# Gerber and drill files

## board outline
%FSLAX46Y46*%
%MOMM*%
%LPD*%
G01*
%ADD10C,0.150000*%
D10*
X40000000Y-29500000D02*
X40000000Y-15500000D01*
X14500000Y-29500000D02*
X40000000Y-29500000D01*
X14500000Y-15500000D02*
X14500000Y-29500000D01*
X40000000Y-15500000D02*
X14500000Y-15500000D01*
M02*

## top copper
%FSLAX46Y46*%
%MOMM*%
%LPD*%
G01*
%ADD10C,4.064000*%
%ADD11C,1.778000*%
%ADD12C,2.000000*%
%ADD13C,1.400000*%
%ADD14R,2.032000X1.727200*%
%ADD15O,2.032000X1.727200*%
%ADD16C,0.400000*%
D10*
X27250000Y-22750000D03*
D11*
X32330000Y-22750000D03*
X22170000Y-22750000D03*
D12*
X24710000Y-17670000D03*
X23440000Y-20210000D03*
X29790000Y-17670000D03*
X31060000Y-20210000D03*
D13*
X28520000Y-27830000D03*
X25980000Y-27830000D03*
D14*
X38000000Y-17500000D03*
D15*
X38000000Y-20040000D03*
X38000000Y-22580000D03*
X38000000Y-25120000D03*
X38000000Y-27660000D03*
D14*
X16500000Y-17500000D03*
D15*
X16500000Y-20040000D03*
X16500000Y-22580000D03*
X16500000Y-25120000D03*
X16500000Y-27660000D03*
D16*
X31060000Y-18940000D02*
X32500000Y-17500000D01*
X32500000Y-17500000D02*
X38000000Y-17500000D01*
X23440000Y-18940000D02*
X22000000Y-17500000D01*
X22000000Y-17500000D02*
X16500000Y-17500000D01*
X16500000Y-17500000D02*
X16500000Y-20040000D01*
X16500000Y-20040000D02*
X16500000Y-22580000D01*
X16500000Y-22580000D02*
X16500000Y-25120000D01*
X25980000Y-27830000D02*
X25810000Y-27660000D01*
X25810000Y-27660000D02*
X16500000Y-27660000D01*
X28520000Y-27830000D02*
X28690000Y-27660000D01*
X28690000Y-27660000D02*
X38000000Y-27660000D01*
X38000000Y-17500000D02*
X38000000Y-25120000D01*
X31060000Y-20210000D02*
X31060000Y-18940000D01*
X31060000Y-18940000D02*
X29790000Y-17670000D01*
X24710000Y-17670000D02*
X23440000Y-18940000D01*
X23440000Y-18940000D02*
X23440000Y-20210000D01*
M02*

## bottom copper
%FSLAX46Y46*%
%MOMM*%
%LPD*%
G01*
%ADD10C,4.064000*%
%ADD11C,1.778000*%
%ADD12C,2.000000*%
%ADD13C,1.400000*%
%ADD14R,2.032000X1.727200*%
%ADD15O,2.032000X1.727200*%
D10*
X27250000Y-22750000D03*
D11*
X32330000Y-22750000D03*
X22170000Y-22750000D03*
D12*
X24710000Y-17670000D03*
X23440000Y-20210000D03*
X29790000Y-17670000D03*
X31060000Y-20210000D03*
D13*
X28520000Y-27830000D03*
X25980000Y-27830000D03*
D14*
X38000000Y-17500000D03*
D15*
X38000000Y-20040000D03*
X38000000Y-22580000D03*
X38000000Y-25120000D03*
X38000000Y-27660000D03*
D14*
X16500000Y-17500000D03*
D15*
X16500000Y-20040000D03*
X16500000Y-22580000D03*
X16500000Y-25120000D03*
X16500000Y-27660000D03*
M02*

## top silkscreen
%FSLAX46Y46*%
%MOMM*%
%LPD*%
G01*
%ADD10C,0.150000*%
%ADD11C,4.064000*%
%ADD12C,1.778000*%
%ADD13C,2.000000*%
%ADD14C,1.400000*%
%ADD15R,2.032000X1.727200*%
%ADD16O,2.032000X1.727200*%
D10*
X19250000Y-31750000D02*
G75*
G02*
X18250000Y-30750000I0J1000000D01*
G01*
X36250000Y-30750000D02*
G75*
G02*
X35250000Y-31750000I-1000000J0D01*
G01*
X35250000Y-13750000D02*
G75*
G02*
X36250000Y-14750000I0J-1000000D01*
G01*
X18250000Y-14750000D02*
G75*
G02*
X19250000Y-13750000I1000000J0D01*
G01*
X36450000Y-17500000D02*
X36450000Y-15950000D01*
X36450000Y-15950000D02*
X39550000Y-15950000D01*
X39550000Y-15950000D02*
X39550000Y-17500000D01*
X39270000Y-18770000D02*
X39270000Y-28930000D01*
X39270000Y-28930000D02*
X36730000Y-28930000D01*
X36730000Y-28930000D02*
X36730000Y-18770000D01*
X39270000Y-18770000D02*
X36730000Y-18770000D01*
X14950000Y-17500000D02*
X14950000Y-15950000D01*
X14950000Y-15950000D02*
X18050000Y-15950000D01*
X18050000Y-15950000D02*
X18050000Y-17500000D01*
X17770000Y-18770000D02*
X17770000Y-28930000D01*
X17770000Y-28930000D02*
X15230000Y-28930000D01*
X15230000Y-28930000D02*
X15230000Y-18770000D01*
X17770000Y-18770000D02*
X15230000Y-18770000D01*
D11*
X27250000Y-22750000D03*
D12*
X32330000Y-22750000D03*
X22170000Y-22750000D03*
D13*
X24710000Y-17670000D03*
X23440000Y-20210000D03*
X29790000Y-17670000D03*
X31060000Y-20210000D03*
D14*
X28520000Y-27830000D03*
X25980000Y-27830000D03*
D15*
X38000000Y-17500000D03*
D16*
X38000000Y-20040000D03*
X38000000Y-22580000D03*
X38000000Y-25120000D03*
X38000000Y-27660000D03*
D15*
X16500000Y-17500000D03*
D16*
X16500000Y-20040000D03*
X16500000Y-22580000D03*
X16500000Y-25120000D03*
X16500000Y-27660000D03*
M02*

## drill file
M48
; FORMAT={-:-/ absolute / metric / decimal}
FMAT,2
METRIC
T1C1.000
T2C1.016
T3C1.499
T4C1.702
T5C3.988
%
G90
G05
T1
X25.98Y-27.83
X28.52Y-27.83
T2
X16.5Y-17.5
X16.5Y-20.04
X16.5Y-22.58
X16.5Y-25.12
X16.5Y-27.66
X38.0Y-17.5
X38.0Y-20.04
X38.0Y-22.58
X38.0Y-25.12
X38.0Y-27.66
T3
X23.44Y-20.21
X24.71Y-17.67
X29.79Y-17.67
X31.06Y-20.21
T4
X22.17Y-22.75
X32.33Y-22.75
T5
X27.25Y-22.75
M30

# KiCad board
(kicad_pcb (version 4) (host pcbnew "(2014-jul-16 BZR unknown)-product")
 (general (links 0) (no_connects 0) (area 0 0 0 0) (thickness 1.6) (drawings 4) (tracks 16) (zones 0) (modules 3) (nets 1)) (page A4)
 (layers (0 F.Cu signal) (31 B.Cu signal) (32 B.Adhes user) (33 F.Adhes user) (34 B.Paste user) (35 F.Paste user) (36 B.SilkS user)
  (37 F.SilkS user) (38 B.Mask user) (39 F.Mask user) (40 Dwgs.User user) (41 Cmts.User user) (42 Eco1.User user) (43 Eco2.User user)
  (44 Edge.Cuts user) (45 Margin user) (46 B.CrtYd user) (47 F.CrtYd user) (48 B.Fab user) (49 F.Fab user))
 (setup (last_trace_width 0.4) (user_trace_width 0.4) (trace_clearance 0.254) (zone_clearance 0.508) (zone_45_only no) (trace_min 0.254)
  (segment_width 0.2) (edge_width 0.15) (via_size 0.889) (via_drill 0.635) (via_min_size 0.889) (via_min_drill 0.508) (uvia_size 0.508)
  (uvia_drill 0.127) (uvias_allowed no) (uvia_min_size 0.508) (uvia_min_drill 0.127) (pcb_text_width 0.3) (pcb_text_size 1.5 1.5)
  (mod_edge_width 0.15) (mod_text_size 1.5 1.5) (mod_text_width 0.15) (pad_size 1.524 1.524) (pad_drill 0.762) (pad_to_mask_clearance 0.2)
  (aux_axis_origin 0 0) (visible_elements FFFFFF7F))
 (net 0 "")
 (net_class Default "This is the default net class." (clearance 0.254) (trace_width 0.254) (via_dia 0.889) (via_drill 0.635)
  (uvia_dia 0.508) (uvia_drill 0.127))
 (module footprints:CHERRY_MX (layer F.Cu) (at 27.25 22.75)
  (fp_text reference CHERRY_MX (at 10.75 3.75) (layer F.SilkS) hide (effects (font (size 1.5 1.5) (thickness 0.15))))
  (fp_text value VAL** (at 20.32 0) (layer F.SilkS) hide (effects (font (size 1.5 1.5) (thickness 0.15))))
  (fp_arc (start -8 8) (end -8 9) (angle 90) (layer F.SilkS) (width 0.15))
  (fp_arc (start 8 8) (end 9 8) (angle 90) (layer F.SilkS) (width 0.15))
  (fp_arc (start 8 -8) (end 8 -9) (angle 90) (layer F.SilkS) (width 0.15))
  (fp_arc (start -8 -8) (end -9 -8) (angle 90) (layer F.SilkS) (width 0.15))
  (pad "" thru_hole circle (at 0 0) (size 4.064 4.064) (drill 3.9878) (layers *.Cu *.Mask F.SilkS))
  (pad "" thru_hole circle (at 5.08 0) (size 1.778 1.778) (drill 1.7018) (layers *.Cu *.Mask F.SilkS))
  (pad "" thru_hole circle (at -5.08 0) (size 1.778 1.778) (drill 1.7018) (layers *.Cu *.Mask F.SilkS))
  (pad 1 thru_hole circle (at -2.54 -5.08) (size 2 2) (drill 1.4986) (layers *.Cu *.Mask F.SilkS))
  (pad 1 thru_hole circle (at -3.81 -2.54) (size 2 2) (drill 1.4986) (layers *.Cu *.Mask F.SilkS))
  (pad 2 thru_hole circle (at 2.54 -5.08) (size 2 2) (drill 1.4986) (layers *.Cu *.Mask F.SilkS))
  (pad 2 thru_hole circle (at 3.81 -2.54) (size 2 2) (drill 1.4986) (layers *.Cu *.Mask F.SilkS))
  (pad 4 thru_hole circle (at 1.27 5.08) (size 1.4 1.4) (drill 1) (layers *.Cu *.Mask F.SilkS))
  (pad 3 thru_hole circle (at -1.27 5.08) (size 1.4 1.4) (drill 1) (layers *.Cu *.Mask F.SilkS)))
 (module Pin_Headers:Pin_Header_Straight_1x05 (layer F.Cu) (at 38 17.5)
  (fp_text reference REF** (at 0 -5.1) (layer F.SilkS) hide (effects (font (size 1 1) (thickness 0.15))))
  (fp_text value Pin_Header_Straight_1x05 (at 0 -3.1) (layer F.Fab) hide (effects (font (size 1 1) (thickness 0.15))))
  (fp_line (start -1.55 0) (end -1.55 -1.55) (layer F.SilkS) (width 0.15))
  (fp_line (start -1.55 -1.55) (end 1.55 -1.55) (layer F.SilkS) (width 0.15))
  (fp_line (start 1.55 -1.55) (end 1.55 0) (layer F.SilkS) (width 0.15))
  (fp_line (start 1.27 1.27) (end 1.27 11.43) (layer F.SilkS) (width 0.15))
  (fp_line (start 1.27 11.43) (end -1.27 11.43) (layer F.SilkS) (width 0.15))
  (fp_line (start -1.27 11.43) (end -1.27 1.27) (layer F.SilkS) (width 0.15))
  (fp_line (start 1.27 1.27) (end -1.27 1.27) (layer F.SilkS) (width 0.15))
  (pad 1 thru_hole rect (at 0 0) (size 2.032 1.7272) (drill 1.016) (layers *.Cu *.Mask F.SilkS))
  (pad 2 thru_hole oval (at 0 2.54) (size 2.032 1.7272) (drill 1.016) (layers *.Cu *.Mask F.SilkS))
  (pad 3 thru_hole oval (at 0 5.08) (size 2.032 1.7272) (drill 1.016) (layers *.Cu *.Mask F.SilkS))
  (pad 4 thru_hole oval (at 0 7.62) (size 2.032 1.7272) (drill 1.016) (layers *.Cu *.Mask F.SilkS))
  (pad 5 thru_hole oval (at 0 10.16) (size 2.032 1.7272) (drill 1.016) (layers *.Cu *.Mask F.SilkS)))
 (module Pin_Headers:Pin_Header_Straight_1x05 (layer F.Cu) (at 16.5 17.5)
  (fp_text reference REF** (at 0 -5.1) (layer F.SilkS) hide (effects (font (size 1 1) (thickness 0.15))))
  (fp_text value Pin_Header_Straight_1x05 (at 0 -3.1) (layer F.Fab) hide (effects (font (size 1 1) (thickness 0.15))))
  (fp_line (start -1.55 0) (end -1.55 -1.55) (layer F.SilkS) (width 0.15))
  (fp_line (start -1.55 -1.55) (end 1.55 -1.55) (layer F.SilkS) (width 0.15))
  (fp_line (start 1.55 -1.55) (end 1.55 0) (layer F.SilkS) (width 0.15))
  (fp_line (start 1.27 1.27) (end 1.27 11.43) (layer F.SilkS) (width 0.15))
  (fp_line (start 1.27 11.43) (end -1.27 11.43) (layer F.SilkS) (width 0.15))
  (fp_line (start -1.27 11.43) (end -1.27 1.27) (layer F.SilkS) (width 0.15))
  (fp_line (start 1.27 1.27) (end -1.27 1.27) (layer F.SilkS) (width 0.15))
  (pad 1 thru_hole rect (at 0 0) (size 2.032 1.7272) (drill 1.016) (layers *.Cu *.Mask F.SilkS))
  (pad 2 thru_hole oval (at 0 2.54) (size 2.032 1.7272) (drill 1.016) (layers *.Cu *.Mask F.SilkS))
  (pad 3 thru_hole oval (at 0 5.08) (size 2.032 1.7272) (drill 1.016) (layers *.Cu *.Mask F.SilkS))
  (pad 4 thru_hole oval (at 0 7.62) (size 2.032 1.7272) (drill 1.016) (layers *.Cu *.Mask F.SilkS))
  (pad 5 thru_hole oval (at 0 10.16) (size 2.032 1.7272) (drill 1.016) (layers *.Cu *.Mask F.SilkS)))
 (gr_line (start 40 29.5) (end 40 15.5) (angle 90) (layer Edge.Cuts) (width 0.15))
 (gr_line (start 14.5 29.5) (end 40 29.5) (angle 90) (layer Edge.Cuts) (width 0.15))
 (gr_line (start 14.5 15.5) (end 14.5 29.5) (angle 90) (layer Edge.Cuts) (width 0.15))
 (gr_line (start 40 15.5) (end 14.5 15.5) (angle 90) (layer Edge.Cuts) (width 0.15))
 (segment (start 31.06 18.94) (end 32.5 17.5) (width 0.4) (layer F.Cu) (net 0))
 (segment (start 32.5 17.5) (end 38 17.5) (width 0.4) (layer F.Cu) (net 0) (status 800000))
 (segment (start 23.44 18.94) (end 22 17.5) (width 0.4) (layer F.Cu) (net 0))
 (segment (start 22 17.5) (end 16.5 17.5) (width 0.4) (layer F.Cu) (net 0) (status 800000))
 (segment (start 16.5 17.5) (end 16.5 20.04) (width 0.4) (layer F.Cu) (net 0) (status C00000))
 (segment (start 16.5 20.04) (end 16.5 22.58) (width 0.4) (layer F.Cu) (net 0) (status C00000))
 (segment (start 16.5 22.58) (end 16.5 25.12) (width 0.4) (layer F.Cu) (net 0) (status C00000))
 (segment (start 25.98 27.83) (end 25.81 27.66) (width 0.4) (layer F.Cu) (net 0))
 (segment (start 25.81 27.66) (end 16.5 27.66) (width 0.4) (layer F.Cu) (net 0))
 (segment (start 28.52 27.83) (end 28.69 27.66) (width 0.4) (layer F.Cu) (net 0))
 (segment (start 28.69 27.66) (end 38 27.66) (width 0.4) (layer F.Cu) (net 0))
 (segment (start 38 17.5) (end 38 25.12) (width 0.4) (layer F.Cu) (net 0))
 (segment (start 31.06 20.21) (end 31.06 18.94) (width 0.4) (layer F.Cu) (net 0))
 (segment (start 31.06 18.94) (end 29.79 17.67) (width 0.4) (layer F.Cu) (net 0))
 (segment (start 24.71 17.67) (end 23.44 18.94) (width 0.4) (layer F.Cu) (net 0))
 (segment (start 23.44 18.94) (end 23.44 20.21) (width 0.4) (layer F.Cu) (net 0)))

